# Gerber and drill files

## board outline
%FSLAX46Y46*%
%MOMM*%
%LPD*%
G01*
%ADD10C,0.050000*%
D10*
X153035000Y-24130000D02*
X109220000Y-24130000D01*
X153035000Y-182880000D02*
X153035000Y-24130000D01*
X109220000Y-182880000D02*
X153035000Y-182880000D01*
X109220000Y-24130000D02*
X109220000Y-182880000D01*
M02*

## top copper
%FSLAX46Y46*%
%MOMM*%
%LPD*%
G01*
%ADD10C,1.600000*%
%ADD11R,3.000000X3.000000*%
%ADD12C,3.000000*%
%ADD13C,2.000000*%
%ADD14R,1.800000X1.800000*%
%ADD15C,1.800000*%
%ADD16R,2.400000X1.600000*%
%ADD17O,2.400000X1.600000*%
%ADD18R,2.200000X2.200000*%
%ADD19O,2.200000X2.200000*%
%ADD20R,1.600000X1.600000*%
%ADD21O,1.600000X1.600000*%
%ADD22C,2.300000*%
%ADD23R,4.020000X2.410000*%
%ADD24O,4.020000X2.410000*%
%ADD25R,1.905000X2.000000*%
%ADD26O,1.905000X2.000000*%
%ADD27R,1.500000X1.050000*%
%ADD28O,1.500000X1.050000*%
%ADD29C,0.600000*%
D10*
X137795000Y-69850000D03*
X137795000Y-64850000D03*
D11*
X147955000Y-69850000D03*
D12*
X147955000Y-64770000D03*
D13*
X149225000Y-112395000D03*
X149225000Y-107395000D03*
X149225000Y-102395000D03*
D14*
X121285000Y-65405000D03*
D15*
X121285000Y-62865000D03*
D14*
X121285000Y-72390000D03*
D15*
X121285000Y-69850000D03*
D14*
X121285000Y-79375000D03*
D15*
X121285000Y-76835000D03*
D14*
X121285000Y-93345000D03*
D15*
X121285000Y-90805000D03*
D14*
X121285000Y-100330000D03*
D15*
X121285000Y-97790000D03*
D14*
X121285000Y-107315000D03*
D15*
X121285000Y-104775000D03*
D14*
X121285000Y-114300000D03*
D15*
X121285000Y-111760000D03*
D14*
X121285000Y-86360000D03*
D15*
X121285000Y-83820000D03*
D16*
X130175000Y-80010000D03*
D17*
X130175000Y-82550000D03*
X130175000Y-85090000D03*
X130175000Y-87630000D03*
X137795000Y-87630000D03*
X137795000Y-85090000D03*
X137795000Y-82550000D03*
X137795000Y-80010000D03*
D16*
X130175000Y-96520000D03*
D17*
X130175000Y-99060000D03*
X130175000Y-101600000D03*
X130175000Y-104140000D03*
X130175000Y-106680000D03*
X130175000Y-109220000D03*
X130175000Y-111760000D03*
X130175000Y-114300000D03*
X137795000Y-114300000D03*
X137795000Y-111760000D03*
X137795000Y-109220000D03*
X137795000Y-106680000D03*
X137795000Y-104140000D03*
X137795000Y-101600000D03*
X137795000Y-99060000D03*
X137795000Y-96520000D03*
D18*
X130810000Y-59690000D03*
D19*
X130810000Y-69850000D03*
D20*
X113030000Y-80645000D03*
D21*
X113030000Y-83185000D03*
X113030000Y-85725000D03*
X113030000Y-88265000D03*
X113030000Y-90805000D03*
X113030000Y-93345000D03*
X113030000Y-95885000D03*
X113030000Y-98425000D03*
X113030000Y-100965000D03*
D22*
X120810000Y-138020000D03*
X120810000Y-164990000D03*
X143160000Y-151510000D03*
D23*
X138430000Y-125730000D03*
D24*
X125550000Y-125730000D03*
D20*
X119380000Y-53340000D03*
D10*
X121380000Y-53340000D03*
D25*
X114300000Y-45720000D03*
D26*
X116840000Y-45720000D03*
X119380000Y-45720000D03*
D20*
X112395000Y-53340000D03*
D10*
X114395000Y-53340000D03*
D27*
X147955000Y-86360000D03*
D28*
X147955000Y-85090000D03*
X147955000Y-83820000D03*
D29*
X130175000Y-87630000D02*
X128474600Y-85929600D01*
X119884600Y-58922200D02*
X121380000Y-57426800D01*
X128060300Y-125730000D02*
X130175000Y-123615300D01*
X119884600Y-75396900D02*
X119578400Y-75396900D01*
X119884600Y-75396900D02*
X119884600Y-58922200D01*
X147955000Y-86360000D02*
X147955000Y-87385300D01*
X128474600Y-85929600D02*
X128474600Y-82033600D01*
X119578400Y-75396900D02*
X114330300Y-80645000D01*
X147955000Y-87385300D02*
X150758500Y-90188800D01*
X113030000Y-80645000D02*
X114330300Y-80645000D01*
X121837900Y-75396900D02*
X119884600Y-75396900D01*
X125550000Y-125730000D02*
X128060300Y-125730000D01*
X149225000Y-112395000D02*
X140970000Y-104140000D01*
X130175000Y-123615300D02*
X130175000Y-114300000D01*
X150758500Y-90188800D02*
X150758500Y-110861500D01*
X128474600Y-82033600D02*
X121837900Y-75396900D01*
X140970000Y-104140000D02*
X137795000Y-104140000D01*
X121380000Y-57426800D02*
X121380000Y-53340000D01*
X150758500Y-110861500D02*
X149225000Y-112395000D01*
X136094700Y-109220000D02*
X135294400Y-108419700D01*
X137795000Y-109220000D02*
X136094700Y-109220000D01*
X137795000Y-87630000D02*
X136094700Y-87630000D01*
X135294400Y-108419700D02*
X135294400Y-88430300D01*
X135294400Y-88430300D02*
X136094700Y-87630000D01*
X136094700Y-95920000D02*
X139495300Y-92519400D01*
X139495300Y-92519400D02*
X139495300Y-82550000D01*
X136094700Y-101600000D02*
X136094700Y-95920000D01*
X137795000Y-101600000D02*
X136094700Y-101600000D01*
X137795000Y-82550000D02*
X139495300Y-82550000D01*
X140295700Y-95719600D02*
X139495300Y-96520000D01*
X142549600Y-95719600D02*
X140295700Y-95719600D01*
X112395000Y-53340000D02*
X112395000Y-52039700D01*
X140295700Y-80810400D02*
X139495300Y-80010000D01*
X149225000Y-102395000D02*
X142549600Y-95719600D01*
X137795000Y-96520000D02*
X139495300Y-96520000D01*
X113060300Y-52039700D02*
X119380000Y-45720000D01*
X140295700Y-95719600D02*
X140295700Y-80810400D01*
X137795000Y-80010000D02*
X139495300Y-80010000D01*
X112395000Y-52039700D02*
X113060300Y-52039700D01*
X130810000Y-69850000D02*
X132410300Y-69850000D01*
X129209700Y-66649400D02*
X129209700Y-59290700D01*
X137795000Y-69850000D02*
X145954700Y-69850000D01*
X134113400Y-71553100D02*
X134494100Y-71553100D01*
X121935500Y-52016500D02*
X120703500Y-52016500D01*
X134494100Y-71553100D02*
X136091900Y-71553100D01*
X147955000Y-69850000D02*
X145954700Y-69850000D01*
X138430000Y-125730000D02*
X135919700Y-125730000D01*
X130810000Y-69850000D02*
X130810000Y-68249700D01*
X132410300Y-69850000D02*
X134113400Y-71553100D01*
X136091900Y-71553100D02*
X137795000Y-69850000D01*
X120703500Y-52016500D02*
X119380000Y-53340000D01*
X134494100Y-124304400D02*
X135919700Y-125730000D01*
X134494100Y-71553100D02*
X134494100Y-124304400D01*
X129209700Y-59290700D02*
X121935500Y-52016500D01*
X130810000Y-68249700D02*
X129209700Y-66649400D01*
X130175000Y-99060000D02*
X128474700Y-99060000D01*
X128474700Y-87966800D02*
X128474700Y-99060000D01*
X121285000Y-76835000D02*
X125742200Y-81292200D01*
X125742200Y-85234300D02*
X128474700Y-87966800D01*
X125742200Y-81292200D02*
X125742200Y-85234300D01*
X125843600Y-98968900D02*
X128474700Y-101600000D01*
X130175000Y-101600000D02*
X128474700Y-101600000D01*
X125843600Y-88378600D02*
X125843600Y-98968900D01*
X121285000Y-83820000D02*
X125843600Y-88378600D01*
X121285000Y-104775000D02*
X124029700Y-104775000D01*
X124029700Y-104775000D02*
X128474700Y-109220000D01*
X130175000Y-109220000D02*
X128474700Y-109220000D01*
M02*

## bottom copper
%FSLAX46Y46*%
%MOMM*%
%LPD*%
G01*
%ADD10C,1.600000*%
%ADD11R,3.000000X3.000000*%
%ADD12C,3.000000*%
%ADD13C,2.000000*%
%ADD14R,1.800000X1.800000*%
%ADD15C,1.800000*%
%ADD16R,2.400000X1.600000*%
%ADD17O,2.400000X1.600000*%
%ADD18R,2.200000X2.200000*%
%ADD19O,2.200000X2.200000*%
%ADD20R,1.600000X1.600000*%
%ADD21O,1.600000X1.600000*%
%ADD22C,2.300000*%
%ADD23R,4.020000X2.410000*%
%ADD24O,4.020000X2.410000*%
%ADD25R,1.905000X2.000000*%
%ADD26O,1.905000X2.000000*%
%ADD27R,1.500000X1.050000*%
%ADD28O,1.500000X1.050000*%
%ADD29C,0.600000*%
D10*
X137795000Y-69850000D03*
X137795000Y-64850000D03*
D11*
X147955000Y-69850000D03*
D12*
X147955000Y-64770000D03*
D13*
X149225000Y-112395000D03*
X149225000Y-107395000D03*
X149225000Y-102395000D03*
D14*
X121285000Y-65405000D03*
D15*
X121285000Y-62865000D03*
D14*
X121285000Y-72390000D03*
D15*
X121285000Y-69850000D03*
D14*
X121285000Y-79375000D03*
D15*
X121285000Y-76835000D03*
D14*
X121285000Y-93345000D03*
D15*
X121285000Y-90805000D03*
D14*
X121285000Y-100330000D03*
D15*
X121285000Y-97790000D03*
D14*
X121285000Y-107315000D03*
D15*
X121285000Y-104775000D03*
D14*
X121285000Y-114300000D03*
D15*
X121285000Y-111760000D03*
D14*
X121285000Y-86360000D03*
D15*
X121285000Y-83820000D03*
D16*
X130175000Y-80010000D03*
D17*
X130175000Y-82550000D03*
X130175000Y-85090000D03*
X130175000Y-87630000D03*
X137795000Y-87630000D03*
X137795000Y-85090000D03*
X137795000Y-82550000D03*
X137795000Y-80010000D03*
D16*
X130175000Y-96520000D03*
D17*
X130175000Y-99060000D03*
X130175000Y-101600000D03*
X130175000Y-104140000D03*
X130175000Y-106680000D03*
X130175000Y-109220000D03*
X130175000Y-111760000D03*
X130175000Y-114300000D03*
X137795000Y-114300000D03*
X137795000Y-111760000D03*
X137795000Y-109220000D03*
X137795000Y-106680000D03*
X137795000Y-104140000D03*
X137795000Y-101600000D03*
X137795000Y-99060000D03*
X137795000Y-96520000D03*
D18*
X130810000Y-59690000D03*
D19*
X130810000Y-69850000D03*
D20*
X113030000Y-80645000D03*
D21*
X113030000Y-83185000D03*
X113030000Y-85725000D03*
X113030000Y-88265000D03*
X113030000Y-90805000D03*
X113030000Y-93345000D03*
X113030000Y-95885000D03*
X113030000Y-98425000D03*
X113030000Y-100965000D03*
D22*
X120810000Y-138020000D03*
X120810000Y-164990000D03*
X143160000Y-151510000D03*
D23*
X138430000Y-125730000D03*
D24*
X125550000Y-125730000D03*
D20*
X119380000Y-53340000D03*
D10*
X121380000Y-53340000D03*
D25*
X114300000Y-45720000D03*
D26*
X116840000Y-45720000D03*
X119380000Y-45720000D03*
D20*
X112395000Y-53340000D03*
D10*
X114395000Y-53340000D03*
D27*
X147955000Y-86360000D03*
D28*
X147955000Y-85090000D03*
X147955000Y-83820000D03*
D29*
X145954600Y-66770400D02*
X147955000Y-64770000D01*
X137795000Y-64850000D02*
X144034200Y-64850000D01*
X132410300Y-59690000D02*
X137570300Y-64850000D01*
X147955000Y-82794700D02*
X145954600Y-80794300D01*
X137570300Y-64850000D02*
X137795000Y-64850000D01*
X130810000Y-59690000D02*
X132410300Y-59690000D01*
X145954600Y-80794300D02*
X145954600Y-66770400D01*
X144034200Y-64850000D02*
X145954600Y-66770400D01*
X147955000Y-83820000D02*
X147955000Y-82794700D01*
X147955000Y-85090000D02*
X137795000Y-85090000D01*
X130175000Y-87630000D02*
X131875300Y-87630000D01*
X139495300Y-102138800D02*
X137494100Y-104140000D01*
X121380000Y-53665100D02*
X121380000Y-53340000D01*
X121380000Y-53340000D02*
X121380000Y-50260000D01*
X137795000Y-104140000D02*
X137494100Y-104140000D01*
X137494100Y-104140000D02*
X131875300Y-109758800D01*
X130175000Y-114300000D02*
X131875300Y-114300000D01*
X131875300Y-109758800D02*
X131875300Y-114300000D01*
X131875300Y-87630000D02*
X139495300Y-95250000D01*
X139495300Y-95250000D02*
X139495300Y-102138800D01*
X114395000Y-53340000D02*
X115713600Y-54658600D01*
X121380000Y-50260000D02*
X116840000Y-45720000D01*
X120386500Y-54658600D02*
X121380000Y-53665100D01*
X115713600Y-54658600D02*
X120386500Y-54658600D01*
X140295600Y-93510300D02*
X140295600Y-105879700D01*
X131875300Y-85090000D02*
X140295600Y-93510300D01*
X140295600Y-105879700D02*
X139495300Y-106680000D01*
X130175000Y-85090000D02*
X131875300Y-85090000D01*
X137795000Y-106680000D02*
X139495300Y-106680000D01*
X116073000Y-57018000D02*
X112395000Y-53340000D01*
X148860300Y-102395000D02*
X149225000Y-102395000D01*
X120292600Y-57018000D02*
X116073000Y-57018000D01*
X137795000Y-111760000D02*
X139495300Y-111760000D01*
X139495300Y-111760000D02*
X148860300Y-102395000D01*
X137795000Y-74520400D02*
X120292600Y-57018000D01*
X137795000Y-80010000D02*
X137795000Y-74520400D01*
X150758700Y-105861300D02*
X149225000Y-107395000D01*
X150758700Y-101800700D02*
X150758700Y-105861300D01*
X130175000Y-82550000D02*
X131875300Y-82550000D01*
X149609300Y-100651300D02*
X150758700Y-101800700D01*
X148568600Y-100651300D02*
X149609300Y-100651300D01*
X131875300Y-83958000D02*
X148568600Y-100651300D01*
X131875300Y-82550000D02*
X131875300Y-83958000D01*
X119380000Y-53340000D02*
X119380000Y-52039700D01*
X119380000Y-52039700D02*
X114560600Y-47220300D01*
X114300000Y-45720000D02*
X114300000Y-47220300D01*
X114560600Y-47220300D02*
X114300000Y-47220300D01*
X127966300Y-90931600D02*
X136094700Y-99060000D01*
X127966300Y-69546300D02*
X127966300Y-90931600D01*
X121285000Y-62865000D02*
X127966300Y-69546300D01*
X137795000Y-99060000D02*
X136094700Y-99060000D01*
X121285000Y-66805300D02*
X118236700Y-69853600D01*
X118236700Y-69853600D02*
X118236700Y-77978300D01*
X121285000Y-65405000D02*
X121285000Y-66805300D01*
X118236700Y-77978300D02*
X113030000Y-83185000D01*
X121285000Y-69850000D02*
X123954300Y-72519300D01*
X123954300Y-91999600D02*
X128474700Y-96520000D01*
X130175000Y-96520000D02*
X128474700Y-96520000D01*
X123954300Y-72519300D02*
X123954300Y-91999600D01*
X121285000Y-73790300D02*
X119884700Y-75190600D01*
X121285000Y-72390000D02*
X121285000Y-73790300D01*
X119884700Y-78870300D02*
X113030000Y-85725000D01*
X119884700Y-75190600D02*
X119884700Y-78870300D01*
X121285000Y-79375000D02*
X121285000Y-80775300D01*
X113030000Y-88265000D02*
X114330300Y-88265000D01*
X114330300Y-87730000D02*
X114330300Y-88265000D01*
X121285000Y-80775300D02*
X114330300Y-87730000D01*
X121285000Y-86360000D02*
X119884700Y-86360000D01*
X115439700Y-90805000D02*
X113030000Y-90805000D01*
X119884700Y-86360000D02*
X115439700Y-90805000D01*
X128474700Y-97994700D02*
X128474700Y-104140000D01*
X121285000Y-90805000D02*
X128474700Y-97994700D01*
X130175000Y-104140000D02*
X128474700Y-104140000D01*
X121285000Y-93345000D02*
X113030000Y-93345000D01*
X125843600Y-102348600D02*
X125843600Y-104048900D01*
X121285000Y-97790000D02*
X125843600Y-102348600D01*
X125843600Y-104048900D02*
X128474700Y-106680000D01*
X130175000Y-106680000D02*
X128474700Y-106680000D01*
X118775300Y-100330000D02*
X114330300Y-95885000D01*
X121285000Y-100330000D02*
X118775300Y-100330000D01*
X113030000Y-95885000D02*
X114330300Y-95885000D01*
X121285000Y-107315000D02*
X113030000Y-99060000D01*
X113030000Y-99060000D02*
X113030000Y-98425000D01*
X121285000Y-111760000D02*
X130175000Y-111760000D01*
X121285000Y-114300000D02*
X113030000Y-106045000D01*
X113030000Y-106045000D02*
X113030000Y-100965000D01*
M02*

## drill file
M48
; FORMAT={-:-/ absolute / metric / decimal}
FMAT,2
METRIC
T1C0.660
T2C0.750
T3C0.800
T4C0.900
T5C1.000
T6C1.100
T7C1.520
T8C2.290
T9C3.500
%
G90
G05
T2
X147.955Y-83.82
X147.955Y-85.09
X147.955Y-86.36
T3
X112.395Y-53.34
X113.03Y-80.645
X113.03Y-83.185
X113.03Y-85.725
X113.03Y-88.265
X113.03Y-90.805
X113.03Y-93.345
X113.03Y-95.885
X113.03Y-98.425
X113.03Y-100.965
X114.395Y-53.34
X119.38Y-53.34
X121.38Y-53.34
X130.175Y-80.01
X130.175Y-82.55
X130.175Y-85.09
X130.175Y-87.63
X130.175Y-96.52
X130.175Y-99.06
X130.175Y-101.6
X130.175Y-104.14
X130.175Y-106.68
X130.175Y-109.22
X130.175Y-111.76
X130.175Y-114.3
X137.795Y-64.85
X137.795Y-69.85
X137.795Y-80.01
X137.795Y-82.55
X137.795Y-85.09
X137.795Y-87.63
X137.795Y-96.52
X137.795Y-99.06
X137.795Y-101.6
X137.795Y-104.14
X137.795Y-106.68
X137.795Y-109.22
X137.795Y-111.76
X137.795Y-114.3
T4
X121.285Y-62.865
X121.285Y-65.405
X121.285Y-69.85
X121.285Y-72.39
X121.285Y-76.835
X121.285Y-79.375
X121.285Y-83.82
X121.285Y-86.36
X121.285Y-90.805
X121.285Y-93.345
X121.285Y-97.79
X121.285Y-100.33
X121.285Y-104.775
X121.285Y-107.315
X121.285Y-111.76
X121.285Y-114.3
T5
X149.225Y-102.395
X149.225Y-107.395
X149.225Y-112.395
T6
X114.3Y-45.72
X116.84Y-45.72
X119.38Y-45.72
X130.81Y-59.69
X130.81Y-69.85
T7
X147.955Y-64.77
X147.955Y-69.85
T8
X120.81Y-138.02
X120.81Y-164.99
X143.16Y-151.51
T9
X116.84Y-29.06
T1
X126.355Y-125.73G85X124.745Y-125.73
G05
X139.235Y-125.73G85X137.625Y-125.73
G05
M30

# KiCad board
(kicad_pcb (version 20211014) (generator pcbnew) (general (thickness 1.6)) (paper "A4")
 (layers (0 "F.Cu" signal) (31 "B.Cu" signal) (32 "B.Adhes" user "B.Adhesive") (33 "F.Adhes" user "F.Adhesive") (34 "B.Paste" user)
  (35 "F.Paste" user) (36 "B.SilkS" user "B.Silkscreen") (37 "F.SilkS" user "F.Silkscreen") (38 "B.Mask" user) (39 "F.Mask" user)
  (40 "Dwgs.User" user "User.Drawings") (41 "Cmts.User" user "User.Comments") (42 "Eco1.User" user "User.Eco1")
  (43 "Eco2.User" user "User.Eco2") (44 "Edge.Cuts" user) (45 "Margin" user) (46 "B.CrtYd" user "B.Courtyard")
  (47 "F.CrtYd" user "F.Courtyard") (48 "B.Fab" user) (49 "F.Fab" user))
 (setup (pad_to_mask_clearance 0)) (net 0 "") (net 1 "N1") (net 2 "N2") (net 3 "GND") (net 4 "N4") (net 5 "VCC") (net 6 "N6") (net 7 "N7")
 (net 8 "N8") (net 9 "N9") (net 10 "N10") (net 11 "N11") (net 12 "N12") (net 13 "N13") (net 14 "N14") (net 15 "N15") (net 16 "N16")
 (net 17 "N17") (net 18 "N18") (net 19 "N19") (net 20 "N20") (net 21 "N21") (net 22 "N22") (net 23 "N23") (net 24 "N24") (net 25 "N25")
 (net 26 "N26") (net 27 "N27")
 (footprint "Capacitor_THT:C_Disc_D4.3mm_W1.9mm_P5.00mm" (layer "F.Cu") (at 137.795 69.85 90)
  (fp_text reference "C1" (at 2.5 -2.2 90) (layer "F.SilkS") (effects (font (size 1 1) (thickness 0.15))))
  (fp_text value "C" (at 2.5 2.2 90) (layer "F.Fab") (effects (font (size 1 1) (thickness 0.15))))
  (pad "1" thru_hole circle locked (at 0 0 90) (size 1.6 1.6) (drill 0.8) (layers *.Cu *.Mask) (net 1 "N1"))
  (pad "2" thru_hole circle locked (at 5 0 90) (size 1.6 1.6) (drill 0.8) (layers *.Cu *.Mask) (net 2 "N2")))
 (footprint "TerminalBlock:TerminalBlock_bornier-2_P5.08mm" (layer "F.Cu") (at 147.955 69.85 90)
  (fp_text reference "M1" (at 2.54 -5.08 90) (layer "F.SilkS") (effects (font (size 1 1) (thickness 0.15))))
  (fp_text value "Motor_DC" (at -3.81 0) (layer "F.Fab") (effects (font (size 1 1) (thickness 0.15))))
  (pad "1" thru_hole rect locked (at 0 0 90) (size 3 3) (drill 1.52) (layers *.Cu *.Mask) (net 1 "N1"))
  (pad "2" thru_hole circle locked (at 5.08 0 90) (size 3 3) (drill 1.52) (layers *.Cu *.Mask) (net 2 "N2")))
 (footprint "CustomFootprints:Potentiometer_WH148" (layer "F.Cu") (at 140.335 107.395 90)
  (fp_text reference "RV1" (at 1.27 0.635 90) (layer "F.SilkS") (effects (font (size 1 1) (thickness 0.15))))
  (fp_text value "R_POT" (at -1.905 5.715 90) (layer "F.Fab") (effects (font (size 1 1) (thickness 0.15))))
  (pad "1" thru_hole circle locked (at -5 8.89 90) (size 2 2) (drill 1) (layers *.Cu *.Mask) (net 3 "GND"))
  (pad "2" thru_hole circle locked (at 0 8.89 90) (size 2 2) (drill 1) (layers *.Cu *.Mask) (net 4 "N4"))
  (pad "3" thru_hole circle locked (at 5 8.89 90) (size 2 2) (drill 1) (layers *.Cu *.Mask) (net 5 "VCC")))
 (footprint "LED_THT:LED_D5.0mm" (layer "F.Cu") (at 121.285 65.405 90)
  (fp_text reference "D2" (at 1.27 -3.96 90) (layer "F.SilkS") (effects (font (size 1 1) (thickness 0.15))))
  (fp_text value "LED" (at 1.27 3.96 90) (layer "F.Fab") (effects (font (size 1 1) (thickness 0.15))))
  (pad "1" thru_hole rect locked (at 0 0 90) (size 1.8 1.8) (drill 0.9) (layers *.Cu *.Mask) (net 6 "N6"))
  (pad "2" thru_hole circle locked (at 2.54 0 90) (size 1.8 1.8) (drill 0.9) (layers *.Cu *.Mask) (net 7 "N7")))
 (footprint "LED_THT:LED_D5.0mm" (layer "F.Cu") (at 121.285 72.39 90)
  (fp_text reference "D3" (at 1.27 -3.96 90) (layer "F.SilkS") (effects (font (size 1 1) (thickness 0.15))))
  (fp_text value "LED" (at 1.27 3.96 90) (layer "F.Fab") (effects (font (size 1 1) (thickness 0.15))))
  (pad "1" thru_hole rect locked (at 0 0 90) (size 1.8 1.8) (drill 0.9) (layers *.Cu *.Mask) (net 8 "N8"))
  (pad "2" thru_hole circle locked (at 2.54 0 90) (size 1.8 1.8) (drill 0.9) (layers *.Cu *.Mask) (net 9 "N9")))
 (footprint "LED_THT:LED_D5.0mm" (layer "F.Cu") (at 121.285 79.375 90)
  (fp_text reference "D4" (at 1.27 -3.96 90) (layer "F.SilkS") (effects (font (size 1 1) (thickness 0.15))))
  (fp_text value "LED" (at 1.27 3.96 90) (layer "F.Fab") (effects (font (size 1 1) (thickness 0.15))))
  (pad "1" thru_hole rect locked (at 0 0 90) (size 1.8 1.8) (drill 0.9) (layers *.Cu *.Mask) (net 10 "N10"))
  (pad "2" thru_hole circle locked (at 2.54 0 90) (size 1.8 1.8) (drill 0.9) (layers *.Cu *.Mask) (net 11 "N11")))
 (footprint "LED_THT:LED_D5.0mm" (layer "F.Cu") (at 121.285 93.345 90)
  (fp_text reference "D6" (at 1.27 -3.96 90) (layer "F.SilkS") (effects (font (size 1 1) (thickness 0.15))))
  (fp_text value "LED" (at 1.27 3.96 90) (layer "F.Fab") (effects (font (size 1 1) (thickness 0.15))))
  (pad "1" thru_hole rect locked (at 0 0 90) (size 1.8 1.8) (drill 0.9) (layers *.Cu *.Mask) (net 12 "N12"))
  (pad "2" thru_hole circle locked (at 2.54 0 90) (size 1.8 1.8) (drill 0.9) (layers *.Cu *.Mask) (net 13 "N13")))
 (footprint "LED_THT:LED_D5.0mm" (layer "F.Cu") (at 121.285 100.33 90)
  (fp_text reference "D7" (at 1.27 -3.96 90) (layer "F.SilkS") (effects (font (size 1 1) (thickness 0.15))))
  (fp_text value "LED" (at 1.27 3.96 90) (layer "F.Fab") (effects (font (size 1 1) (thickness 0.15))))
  (pad "1" thru_hole rect locked (at 0 0 90) (size 1.8 1.8) (drill 0.9) (layers *.Cu *.Mask) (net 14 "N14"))
  (pad "2" thru_hole circle locked (at 2.54 0 90) (size 1.8 1.8) (drill 0.9) (layers *.Cu *.Mask) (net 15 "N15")))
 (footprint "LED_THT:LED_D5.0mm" (layer "F.Cu") (at 121.285 107.315 90)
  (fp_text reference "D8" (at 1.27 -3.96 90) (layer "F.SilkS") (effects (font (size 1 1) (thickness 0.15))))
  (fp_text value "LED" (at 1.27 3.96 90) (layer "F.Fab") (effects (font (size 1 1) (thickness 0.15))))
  (pad "1" thru_hole rect locked (at 0 0 90) (size 1.8 1.8) (drill 0.9) (layers *.Cu *.Mask) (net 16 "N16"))
  (pad "2" thru_hole circle locked (at 2.54 0 90) (size 1.8 1.8) (drill 0.9) (layers *.Cu *.Mask) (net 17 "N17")))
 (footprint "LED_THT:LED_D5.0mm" (layer "F.Cu") (at 121.285 114.3 90)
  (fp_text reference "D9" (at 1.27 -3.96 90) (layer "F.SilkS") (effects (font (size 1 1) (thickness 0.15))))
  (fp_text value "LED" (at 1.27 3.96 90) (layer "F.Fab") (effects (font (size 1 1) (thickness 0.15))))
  (pad "1" thru_hole rect locked (at 0 0 90) (size 1.8 1.8) (drill 0.9) (layers *.Cu *.Mask) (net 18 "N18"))
  (pad "2" thru_hole circle locked (at 2.54 0 90) (size 1.8 1.8) (drill 0.9) (layers *.Cu *.Mask) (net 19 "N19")))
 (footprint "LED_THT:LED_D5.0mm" (layer "F.Cu") (at 121.285 86.36 90)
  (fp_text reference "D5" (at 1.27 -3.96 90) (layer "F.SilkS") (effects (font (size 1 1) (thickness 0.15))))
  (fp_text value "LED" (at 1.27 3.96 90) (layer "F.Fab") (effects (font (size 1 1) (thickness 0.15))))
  (pad "1" thru_hole rect locked (at 0 0 90) (size 1.8 1.8) (drill 0.9) (layers *.Cu *.Mask) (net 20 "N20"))
  (pad "2" thru_hole circle locked (at 2.54 0 90) (size 1.8 1.8) (drill 0.9) (layers *.Cu *.Mask) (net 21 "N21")))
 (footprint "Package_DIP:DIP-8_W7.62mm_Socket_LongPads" (layer "F.Cu") (at 130.175 80.01)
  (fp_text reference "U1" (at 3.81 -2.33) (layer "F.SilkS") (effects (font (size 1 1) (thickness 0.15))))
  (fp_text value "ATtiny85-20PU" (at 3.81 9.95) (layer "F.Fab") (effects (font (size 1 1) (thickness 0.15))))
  (pad "1" thru_hole rect locked (at 0 0) (size 2.4 1.6) (drill 0.8) (layers *.Cu *.Mask) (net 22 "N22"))
  (pad "2" thru_hole oval locked (at 0 2.54) (size 2.4 1.6) (drill 0.8) (layers *.Cu *.Mask) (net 4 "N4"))
  (pad "3" thru_hole oval locked (at 0 5.08) (size 2.4 1.6) (drill 0.8) (layers *.Cu *.Mask) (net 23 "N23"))
  (pad "4" thru_hole oval locked (at 0 7.62) (size 2.4 1.6) (drill 0.8) (layers *.Cu *.Mask) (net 3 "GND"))
  (pad "5" thru_hole oval locked (at 7.62 7.62) (size 2.4 1.6) (drill 0.8) (layers *.Cu *.Mask) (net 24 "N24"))
  (pad "6" thru_hole oval locked (at 7.62 5.08) (size 2.4 1.6) (drill 0.8) (layers *.Cu *.Mask) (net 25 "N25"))
  (pad "7" thru_hole oval locked (at 7.62 2.54) (size 2.4 1.6) (drill 0.8) (layers *.Cu *.Mask) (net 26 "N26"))
  (pad "8" thru_hole oval locked (at 7.62 0) (size 2.4 1.6) (drill 0.8) (layers *.Cu *.Mask) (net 5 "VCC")))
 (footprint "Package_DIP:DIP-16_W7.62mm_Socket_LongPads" (layer "F.Cu") (at 130.175 96.52)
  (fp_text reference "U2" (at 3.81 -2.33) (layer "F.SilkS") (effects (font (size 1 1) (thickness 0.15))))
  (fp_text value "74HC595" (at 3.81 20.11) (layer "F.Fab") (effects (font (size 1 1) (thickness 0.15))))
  (pad "1" thru_hole rect locked (at 0 0) (size 2.4 1.6) (drill 0.8) (layers *.Cu *.Mask) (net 9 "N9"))
  (pad "2" thru_hole oval locked (at 0 2.54) (size 2.4 1.6) (drill 0.8) (layers *.Cu *.Mask) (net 11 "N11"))
  (pad "3" thru_hole oval locked (at 0 5.08) (size 2.4 1.6) (drill 0.8) (layers *.Cu *.Mask) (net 21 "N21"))
  (pad "4" thru_hole oval locked (at 0 7.62) (size 2.4 1.6) (drill 0.8) (layers *.Cu *.Mask) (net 13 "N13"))
  (pad "5" thru_hole oval locked (at 0 10.16) (size 2.4 1.6) (drill 0.8) (layers *.Cu *.Mask) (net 15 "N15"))
  (pad "6" thru_hole oval locked (at 0 12.7) (size 2.4 1.6) (drill 0.8) (layers *.Cu *.Mask) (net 17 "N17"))
  (pad "7" thru_hole oval locked (at 0 15.24) (size 2.4 1.6) (drill 0.8) (layers *.Cu *.Mask) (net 19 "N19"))
  (pad "8" thru_hole oval locked (at 0 17.78) (size 2.4 1.6) (drill 0.8) (layers *.Cu *.Mask) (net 3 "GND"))
  (pad "9" thru_hole oval locked (at 7.62 17.78) (size 2.4 1.6) (drill 0.8) (layers *.Cu *.Mask) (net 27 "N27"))
  (pad "10" thru_hole oval locked (at 7.62 15.24) (size 2.4 1.6) (drill 0.8) (layers *.Cu *.Mask) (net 5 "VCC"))
  (pad "11" thru_hole oval locked (at 7.62 12.7) (size 2.4 1.6) (drill 0.8) (layers *.Cu *.Mask) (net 24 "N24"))
  (pad "12" thru_hole oval locked (at 7.62 10.16) (size 2.4 1.6) (drill 0.8) (layers *.Cu *.Mask) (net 23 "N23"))
  (pad "13" thru_hole oval locked (at 7.62 7.62) (size 2.4 1.6) (drill 0.8) (layers *.Cu *.Mask) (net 3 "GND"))
  (pad "14" thru_hole oval locked (at 7.62 5.08) (size 2.4 1.6) (drill 0.8) (layers *.Cu *.Mask) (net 26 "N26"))
  (pad "15" thru_hole oval locked (at 7.62 2.54) (size 2.4 1.6) (drill 0.8) (layers *.Cu *.Mask) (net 7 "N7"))
  (pad "16" thru_hole oval locked (at 7.62 0) (size 2.4 1.6) (drill 0.8) (layers *.Cu *.Mask) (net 5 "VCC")))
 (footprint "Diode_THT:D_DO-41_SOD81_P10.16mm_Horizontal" (layer "F.Cu") (at 130.81 59.69 -90)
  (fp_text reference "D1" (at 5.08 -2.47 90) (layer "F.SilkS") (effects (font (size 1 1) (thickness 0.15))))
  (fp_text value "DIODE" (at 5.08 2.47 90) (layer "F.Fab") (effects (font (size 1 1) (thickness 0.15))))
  (pad "1" thru_hole rect locked (at 0 0 270) (size 2.2 2.2) (drill 1.1) (layers *.Cu *.Mask) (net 2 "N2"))
  (pad "2" thru_hole oval locked (at 10.16 0 270) (size 2.2 2.2) (drill 1.1) (layers *.Cu *.Mask) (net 1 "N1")))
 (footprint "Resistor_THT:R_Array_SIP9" (layer "F.Cu") (at 113.03 80.645 -90)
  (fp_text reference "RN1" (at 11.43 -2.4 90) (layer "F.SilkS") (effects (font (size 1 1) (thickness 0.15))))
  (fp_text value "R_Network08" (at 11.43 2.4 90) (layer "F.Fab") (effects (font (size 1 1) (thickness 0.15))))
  (pad "1" thru_hole rect locked (at 0 0 270) (size 1.6 1.6) (drill 0.8) (layers *.Cu *.Mask) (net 3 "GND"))
  (pad "2" thru_hole oval locked (at 2.54 0 270) (size 1.6 1.6) (drill 0.8) (layers *.Cu *.Mask) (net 6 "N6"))
  (pad "3" thru_hole oval locked (at 5.08 0 270) (size 1.6 1.6) (drill 0.8) (layers *.Cu *.Mask) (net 8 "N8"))
  (pad "4" thru_hole oval locked (at 7.62 0 270) (size 1.6 1.6) (drill 0.8) (layers *.Cu *.Mask) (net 10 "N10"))
  (pad "5" thru_hole oval locked (at 10.16 0 270) (size 1.6 1.6) (drill 0.8) (layers *.Cu *.Mask) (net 20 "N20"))
  (pad "6" thru_hole oval locked (at 12.7 0 270) (size 1.6 1.6) (drill 0.8) (layers *.Cu *.Mask) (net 12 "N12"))
  (pad "7" thru_hole oval locked (at 15.24 0 270) (size 1.6 1.6) (drill 0.8) (layers *.Cu *.Mask) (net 14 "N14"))
  (pad "8" thru_hole oval locked (at 17.78 0 270) (size 1.6 1.6) (drill 0.8) (layers *.Cu *.Mask) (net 16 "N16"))
  (pad "9" thru_hole oval locked (at 20.32 0 270) (size 1.6 1.6) (drill 0.8) (layers *.Cu *.Mask) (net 18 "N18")))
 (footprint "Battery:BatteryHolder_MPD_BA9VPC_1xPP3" (layer "F.Cu") (at 138.43 125.73 -90)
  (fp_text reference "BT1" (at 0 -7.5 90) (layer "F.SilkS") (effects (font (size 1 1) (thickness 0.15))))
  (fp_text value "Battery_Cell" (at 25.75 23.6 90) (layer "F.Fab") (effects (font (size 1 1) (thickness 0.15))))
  (pad "" np_thru_hole circle locked (at 12.29 17.62 270) (size 2.3 2.3) (drill 2.29) (layers *.Cu *.Mask))
  (pad "" np_thru_hole circle locked (at 39.26 17.62 270) (size 2.3 2.3) (drill 2.29) (layers *.Cu *.Mask))
  (pad "" np_thru_hole circle locked (at 25.78 -4.73 270) (size 2.3 2.3) (drill 2.29) (layers *.Cu *.Mask))
  (pad "1" thru_hole rect locked (at 0 0 270) (size 2.41 4.02) (drill oval 0.66 2.27) (layers *.Cu *.Mask) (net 1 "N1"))
  (pad "2" thru_hole oval locked (at 0 12.88 270) (size 2.41 4.02) (drill oval 0.66 2.27) (layers *.Cu *.Mask) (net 3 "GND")))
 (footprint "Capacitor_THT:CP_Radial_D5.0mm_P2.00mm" (layer "F.Cu") (at 119.38 53.34)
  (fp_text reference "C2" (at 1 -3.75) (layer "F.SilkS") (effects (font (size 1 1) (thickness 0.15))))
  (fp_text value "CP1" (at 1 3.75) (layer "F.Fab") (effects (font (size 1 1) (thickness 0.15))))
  (pad "1" thru_hole rect locked (at 0 0) (size 1.6 1.6) (drill 0.8) (layers *.Cu *.Mask) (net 1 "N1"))
  (pad "2" thru_hole circle locked (at 2 0) (size 1.6 1.6) (drill 0.8) (layers *.Cu *.Mask) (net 3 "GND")))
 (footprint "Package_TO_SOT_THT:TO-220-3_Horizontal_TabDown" (layer "F.Cu") (at 114.3 45.72)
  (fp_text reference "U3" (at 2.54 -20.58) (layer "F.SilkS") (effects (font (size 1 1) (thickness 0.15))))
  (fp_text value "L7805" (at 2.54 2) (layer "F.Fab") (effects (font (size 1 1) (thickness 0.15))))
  (pad "" np_thru_hole oval locked (at 2.54 -16.66) (size 3.5 3.5) (drill 3.5) (layers *.Cu *.Mask))
  (pad "1" thru_hole rect locked (at 0 0) (size 1.905 2) (drill 1.1) (layers *.Cu *.Mask) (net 1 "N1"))
  (pad "2" thru_hole oval locked (at 2.54 0) (size 1.905 2) (drill 1.1) (layers *.Cu *.Mask) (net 3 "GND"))
  (pad "3" thru_hole oval locked (at 5.08 0) (size 1.905 2) (drill 1.1) (layers *.Cu *.Mask) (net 5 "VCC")))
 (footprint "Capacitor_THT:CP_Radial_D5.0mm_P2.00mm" (layer "F.Cu") (at 112.395 53.34)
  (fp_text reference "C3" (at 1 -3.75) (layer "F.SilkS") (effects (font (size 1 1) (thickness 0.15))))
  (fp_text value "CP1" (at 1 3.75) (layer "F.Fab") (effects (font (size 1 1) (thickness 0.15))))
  (pad "1" thru_hole rect locked (at 0 0) (size 1.6 1.6) (drill 0.8) (layers *.Cu *.Mask) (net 5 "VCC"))
  (pad "2" thru_hole circle locked (at 2 0) (size 1.6 1.6) (drill 0.8) (layers *.Cu *.Mask) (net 3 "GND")))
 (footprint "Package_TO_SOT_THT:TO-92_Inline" (layer "F.Cu") (at 147.955 86.36 90)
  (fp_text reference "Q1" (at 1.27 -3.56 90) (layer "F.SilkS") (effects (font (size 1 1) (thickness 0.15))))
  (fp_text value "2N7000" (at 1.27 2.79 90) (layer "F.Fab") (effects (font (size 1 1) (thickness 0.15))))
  (pad "1" thru_hole rect locked (at 0 0 90) (size 1.05 1.5) (drill 0.75) (layers *.Cu *.Mask) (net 3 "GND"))
  (pad "2" thru_hole oval locked (at 1.27 0 90) (size 1.05 1.5) (drill 0.75) (layers *.Cu *.Mask) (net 25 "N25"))
  (pad "3" thru_hole oval locked (at 2.54 0 90) (size 1.05 1.5) (drill 0.75) (layers *.Cu *.Mask) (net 2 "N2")))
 (gr_line (start 153.035 24.13) (end 109.22 24.13) (layer "Edge.Cuts") (width 0.05))
 (gr_line (start 153.035 182.88) (end 153.035 24.13) (layer "Edge.Cuts") (width 0.05))
 (gr_line (start 109.22 182.88) (end 153.035 182.88) (layer "Edge.Cuts") (width 0.05))
 (gr_line (start 109.22 24.13) (end 109.22 182.88) (layer "Edge.Cuts") (width 0.05))
 (segment (start 145.9546 66.7704) (end 147.955 64.77) (width 0.6) (layer "B.Cu") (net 2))
 (segment (start 137.795 64.85) (end 144.0342 64.85) (width 0.6) (layer "B.Cu") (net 2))
 (segment (start 132.4103 59.69) (end 137.5703 64.85) (width 0.6) (layer "B.Cu") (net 2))
 (segment (start 147.955 82.7947) (end 145.9546 80.7943) (width 0.6) (layer "B.Cu") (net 2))
 (segment (start 137.5703 64.85) (end 137.795 64.85) (width 0.6) (layer "B.Cu") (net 2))
 (segment (start 130.81 59.69) (end 132.4103 59.69) (width 0.6) (layer "B.Cu") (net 2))
 (segment (start 145.9546 80.7943) (end 145.9546 66.7704) (width 0.6) (layer "B.Cu") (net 2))
 (segment (start 144.0342 64.85) (end 145.9546 66.7704) (width 0.6) (layer "B.Cu") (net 2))
 (segment (start 147.955 83.82) (end 147.955 82.7947) (width 0.6) (layer "B.Cu") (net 2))
 (segment (start 147.955 85.09) (end 137.795 85.09) (width 0.6) (layer "B.Cu") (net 25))
 (segment (start 130.175 87.63) (end 128.4746 85.9296) (width 0.6) (layer "F.Cu") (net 3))
 (segment (start 119.8846 58.9222) (end 121.38 57.4268) (width 0.6) (layer "F.Cu") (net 3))
 (segment (start 128.0603 125.73) (end 130.175 123.6153) (width 0.6) (layer "F.Cu") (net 3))
 (segment (start 119.8846 75.3969) (end 119.5784 75.3969) (width 0.6) (layer "F.Cu") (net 3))
 (segment (start 119.8846 75.3969) (end 119.8846 58.9222) (width 0.6) (layer "F.Cu") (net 3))
 (segment (start 147.955 86.36) (end 147.955 87.3853) (width 0.6) (layer "F.Cu") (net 3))
 (segment (start 128.4746 85.9296) (end 128.4746 82.0336) (width 0.6) (layer "F.Cu") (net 3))
 (segment (start 119.5784 75.3969) (end 114.3303 80.645) (width 0.6) (layer "F.Cu") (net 3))
 (segment (start 147.955 87.3853) (end 150.7585 90.1888) (width 0.6) (layer "F.Cu") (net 3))
 (segment (start 113.03 80.645) (end 114.3303 80.645) (width 0.6) (layer "F.Cu") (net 3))
 (segment (start 121.8379 75.3969) (end 119.8846 75.3969) (width 0.6) (layer "F.Cu") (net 3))
 (segment (start 125.55 125.73) (end 128.0603 125.73) (width 0.6) (layer "F.Cu") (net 3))
 (segment (start 149.225 112.395) (end 140.97 104.14) (width 0.6) (layer "F.Cu") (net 3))
 (segment (start 130.175 123.6153) (end 130.175 114.3) (width 0.6) (layer "F.Cu") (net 3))
 (segment (start 150.7585 90.1888) (end 150.7585 110.8615) (width 0.6) (layer "F.Cu") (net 3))
 (segment (start 128.4746 82.0336) (end 121.8379 75.3969) (width 0.6) (layer "F.Cu") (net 3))
 (segment (start 140.97 104.14) (end 137.795 104.14) (width 0.6) (layer "F.Cu") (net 3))
 (segment (start 121.38 57.4268) (end 121.38 53.34) (width 0.6) (layer "F.Cu") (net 3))
 (segment (start 150.7585 110.8615) (end 149.225 112.395) (width 0.6) (layer "F.Cu") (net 3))
 (segment (start 130.175 87.63) (end 131.8753 87.63) (width 0.6) (layer "B.Cu") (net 3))
 (segment (start 139.4953 102.1388) (end 137.4941 104.14) (width 0.6) (layer "B.Cu") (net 3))
 (segment (start 121.38 53.6651) (end 121.38 53.34) (width 0.6) (layer "B.Cu") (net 3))
 (segment (start 121.38 53.34) (end 121.38 50.26) (width 0.6) (layer "B.Cu") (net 3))
 (segment (start 137.795 104.14) (end 137.4941 104.14) (width 0.6) (layer "B.Cu") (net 3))
 (segment (start 137.4941 104.14) (end 131.8753 109.7588) (width 0.6) (layer "B.Cu") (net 3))
 (segment (start 130.175 114.3) (end 131.8753 114.3) (width 0.6) (layer "B.Cu") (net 3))
 (segment (start 131.8753 109.7588) (end 131.8753 114.3) (width 0.6) (layer "B.Cu") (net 3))
 (segment (start 131.8753 87.63) (end 139.4953 95.25) (width 0.6) (layer "B.Cu") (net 3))
 (segment (start 139.4953 95.25) (end 139.4953 102.1388) (width 0.6) (layer "B.Cu") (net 3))
 (segment (start 114.395 53.34) (end 115.7136 54.6586) (width 0.6) (layer "B.Cu") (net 3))
 (segment (start 121.38 50.26) (end 116.84 45.72) (width 0.6) (layer "B.Cu") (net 3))
 (segment (start 120.3865 54.6586) (end 121.38 53.6651) (width 0.6) (layer "B.Cu") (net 3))
 (segment (start 115.7136 54.6586) (end 120.3865 54.6586) (width 0.6) (layer "B.Cu") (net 3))
 (segment (start 136.0947 109.22) (end 135.2944 108.4197) (width 0.6) (layer "F.Cu") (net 24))
 (segment (start 137.795 109.22) (end 136.0947 109.22) (width 0.6) (layer "F.Cu") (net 24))
 (segment (start 137.795 87.63) (end 136.0947 87.63) (width 0.6) (layer "F.Cu") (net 24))
 (segment (start 135.2944 108.4197) (end 135.2944 88.4303) (width 0.6) (layer "F.Cu") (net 24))
 (segment (start 135.2944 88.4303) (end 136.0947 87.63) (width 0.6) (layer "F.Cu") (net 24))
 (segment (start 140.2956 93.5103) (end 140.2956 105.8797) (width 0.6) (layer "B.Cu") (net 23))
 (segment (start 131.8753 85.09) (end 140.2956 93.5103) (width 0.6) (layer "B.Cu") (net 23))
 (segment (start 140.2956 105.8797) (end 139.4953 106.68) (width 0.6) (layer "B.Cu") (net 23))
 (segment (start 130.175 85.09) (end 131.8753 85.09) (width 0.6) (layer "B.Cu") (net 23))
 (segment (start 137.795 106.68) (end 139.4953 106.68) (width 0.6) (layer "B.Cu") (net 23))
 (segment (start 136.0947 95.92) (end 139.4953 92.5194) (width 0.6) (layer "F.Cu") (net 26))
 (segment (start 139.4953 92.5194) (end 139.4953 82.55) (width 0.6) (layer "F.Cu") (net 26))
 (segment (start 136.0947 101.6) (end 136.0947 95.92) (width 0.6) (layer "F.Cu") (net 26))
 (segment (start 137.795 101.6) (end 136.0947 101.6) (width 0.6) (layer "F.Cu") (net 26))
 (segment (start 137.795 82.55) (end 139.4953 82.55) (width 0.6) (layer "F.Cu") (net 26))
 (segment (start 140.2957 95.7196) (end 139.4953 96.52) (width 0.6) (layer "F.Cu") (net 5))
 (segment (start 142.5496 95.7196) (end 140.2957 95.7196) (width 0.6) (layer "F.Cu") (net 5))
 (segment (start 112.395 53.34) (end 112.395 52.0397) (width 0.6) (layer "F.Cu") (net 5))
 (segment (start 140.2957 80.8104) (end 139.4953 80.01) (width 0.6) (layer "F.Cu") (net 5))
 (segment (start 149.225 102.395) (end 142.5496 95.7196) (width 0.6) (layer "F.Cu") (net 5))
 (segment (start 137.795 96.52) (end 139.4953 96.52) (width 0.6) (layer "F.Cu") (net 5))
 (segment (start 113.0603 52.0397) (end 119.38 45.72) (width 0.6) (layer "F.Cu") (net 5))
 (segment (start 140.2957 95.7196) (end 140.2957 80.8104) (width 0.6) (layer "F.Cu") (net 5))
 (segment (start 137.795 80.01) (end 139.4953 80.01) (width 0.6) (layer "F.Cu") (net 5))
 (segment (start 112.395 52.0397) (end 113.0603 52.0397) (width 0.6) (layer "F.Cu") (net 5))
 (segment (start 116.073 57.018) (end 112.395 53.34) (width 0.6) (layer "B.Cu") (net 5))
 (segment (start 148.8603 102.395) (end 149.225 102.395) (width 0.6) (layer "B.Cu") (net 5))
 (segment (start 120.2926 57.018) (end 116.073 57.018) (width 0.6) (layer "B.Cu") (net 5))
 (segment (start 137.795 111.76) (end 139.4953 111.76) (width 0.6) (layer "B.Cu") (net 5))
 (segment (start 139.4953 111.76) (end 148.8603 102.395) (width 0.6) (layer "B.Cu") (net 5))
 (segment (start 137.795 74.5204) (end 120.2926 57.018) (width 0.6) (layer "B.Cu") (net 5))
 (segment (start 137.795 80.01) (end 137.795 74.5204) (width 0.6) (layer "B.Cu") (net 5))
 (segment (start 150.7587 105.8613) (end 149.225 107.395) (width 0.6) (layer "B.Cu") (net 4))
 (segment (start 150.7587 101.8007) (end 150.7587 105.8613) (width 0.6) (layer "B.Cu") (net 4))
 (segment (start 130.175 82.55) (end 131.8753 82.55) (width 0.6) (layer "B.Cu") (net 4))
 (segment (start 149.6093 100.6513) (end 150.7587 101.8007) (width 0.6) (layer "B.Cu") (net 4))
 (segment (start 148.5686 100.6513) (end 149.6093 100.6513) (width 0.6) (layer "B.Cu") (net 4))
 (segment (start 131.8753 83.958) (end 148.5686 100.6513) (width 0.6) (layer "B.Cu") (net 4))
 (segment (start 131.8753 82.55) (end 131.8753 83.958) (width 0.6) (layer "B.Cu") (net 4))
 (segment (start 130.81 69.85) (end 132.4103 69.85) (width 0.6) (layer "F.Cu") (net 1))
 (segment (start 129.2097 66.6494) (end 129.2097 59.2907) (width 0.6) (layer "F.Cu") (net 1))
 (segment (start 137.795 69.85) (end 145.9547 69.85) (width 0.6) (layer "F.Cu") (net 1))
 (segment (start 134.1134 71.5531) (end 134.4941 71.5531) (width 0.6) (layer "F.Cu") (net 1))
 (segment (start 121.9355 52.0165) (end 120.7035 52.0165) (width 0.6) (layer "F.Cu") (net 1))
 (segment (start 134.4941 71.5531) (end 136.0919 71.5531) (width 0.6) (layer "F.Cu") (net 1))
 (segment (start 147.955 69.85) (end 145.9547 69.85) (width 0.6) (layer "F.Cu") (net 1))
 (segment (start 138.43 125.73) (end 135.9197 125.73) (width 0.6) (layer "F.Cu") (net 1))
 (segment (start 130.81 69.85) (end 130.81 68.2497) (width 0.6) (layer "F.Cu") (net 1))
 (segment (start 132.4103 69.85) (end 134.1134 71.5531) (width 0.6) (layer "F.Cu") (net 1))
 (segment (start 136.0919 71.5531) (end 137.795 69.85) (width 0.6) (layer "F.Cu") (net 1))
 (segment (start 120.7035 52.0165) (end 119.38 53.34) (width 0.6) (layer "F.Cu") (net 1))
 (segment (start 134.4941 124.3044) (end 135.9197 125.73) (width 0.6) (layer "F.Cu") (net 1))
 (segment (start 134.4941 71.5531) (end 134.4941 124.3044) (width 0.6) (layer "F.Cu") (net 1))
 (segment (start 129.2097 59.2907) (end 121.9355 52.0165) (width 0.6) (layer "F.Cu") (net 1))
 (segment (start 130.81 68.2497) (end 129.2097 66.6494) (width 0.6) (layer "F.Cu") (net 1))
 (segment (start 119.38 53.34) (end 119.38 52.0397) (width 0.6) (layer "B.Cu") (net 1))
 (segment (start 119.38 52.0397) (end 114.5606 47.2203) (width 0.6) (layer "B.Cu") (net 1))
 (segment (start 114.3 45.72) (end 114.3 47.2203) (width 0.6) (layer "B.Cu") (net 1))
 (segment (start 114.5606 47.2203) (end 114.3 47.2203) (width 0.6) (layer "B.Cu") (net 1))
 (segment (start 127.9663 90.9316) (end 136.0947 99.06) (width 0.6) (layer "B.Cu") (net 7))
 (segment (start 127.9663 69.5463) (end 127.9663 90.9316) (width 0.6) (layer "B.Cu") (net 7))
 (segment (start 121.285 62.865) (end 127.9663 69.5463) (width 0.6) (layer "B.Cu") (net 7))
 (segment (start 137.795 99.06) (end 136.0947 99.06) (width 0.6) (layer "B.Cu") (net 7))
 (segment (start 121.285 66.8053) (end 118.2367 69.8536) (width 0.6) (layer "B.Cu") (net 6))
 (segment (start 118.2367 69.8536) (end 118.2367 77.9783) (width 0.6) (layer "B.Cu") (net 6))
 (segment (start 121.285 65.405) (end 121.285 66.8053) (width 0.6) (layer "B.Cu") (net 6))
 (segment (start 118.2367 77.9783) (end 113.03 83.185) (width 0.6) (layer "B.Cu") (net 6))
 (segment (start 121.285 69.85) (end 123.9543 72.5193) (width 0.6) (layer "B.Cu") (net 9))
 (segment (start 123.9543 91.9996) (end 128.4747 96.52) (width 0.6) (layer "B.Cu") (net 9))
 (segment (start 130.175 96.52) (end 128.4747 96.52) (width 0.6) (layer "B.Cu") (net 9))
 (segment (start 123.9543 72.5193) (end 123.9543 91.9996) (width 0.6) (layer "B.Cu") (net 9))
 (segment (start 121.285 73.7903) (end 119.8847 75.1906) (width 0.6) (layer "B.Cu") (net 8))
 (segment (start 121.285 72.39) (end 121.285 73.7903) (width 0.6) (layer "B.Cu") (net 8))
 (segment (start 119.8847 78.8703) (end 113.03 85.725) (width 0.6) (layer "B.Cu") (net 8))
 (segment (start 119.8847 75.1906) (end 119.8847 78.8703) (width 0.6) (layer "B.Cu") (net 8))
 (segment (start 130.175 99.06) (end 128.4747 99.06) (width 0.6) (layer "F.Cu") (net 11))
 (segment (start 128.4747 87.9668) (end 128.4747 99.06) (width 0.6) (layer "F.Cu") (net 11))
 (segment (start 121.285 76.835) (end 125.7422 81.2922) (width 0.6) (layer "F.Cu") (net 11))
 (segment (start 125.7422 85.2343) (end 128.4747 87.9668) (width 0.6) (layer "F.Cu") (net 11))
 (segment (start 125.7422 81.2922) (end 125.7422 85.2343) (width 0.6) (layer "F.Cu") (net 11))
 (segment (start 121.285 79.375) (end 121.285 80.7753) (width 0.6) (layer "B.Cu") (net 10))
 (segment (start 113.03 88.265) (end 114.3303 88.265) (width 0.6) (layer "B.Cu") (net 10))
 (segment (start 114.3303 87.73) (end 114.3303 88.265) (width 0.6) (layer "B.Cu") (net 10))
 (segment (start 121.285 80.7753) (end 114.3303 87.73) (width 0.6) (layer "B.Cu") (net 10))
 (segment (start 125.8436 98.9689) (end 128.4747 101.6) (width 0.6) (layer "F.Cu") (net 21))
 (segment (start 130.175 101.6) (end 128.4747 101.6) (width 0.6) (layer "F.Cu") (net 21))
 (segment (start 125.8436 88.3786) (end 125.8436 98.9689) (width 0.6) (layer "F.Cu") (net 21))
 (segment (start 121.285 83.82) (end 125.8436 88.3786) (width 0.6) (layer "F.Cu") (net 21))
 (segment (start 121.285 86.36) (end 119.8847 86.36) (width 0.6) (layer "B.Cu") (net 20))
 (segment (start 115.4397 90.805) (end 113.03 90.805) (width 0.6) (layer "B.Cu") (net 20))
 (segment (start 119.8847 86.36) (end 115.4397 90.805) (width 0.6) (layer "B.Cu") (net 20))
 (segment (start 128.4747 97.9947) (end 128.4747 104.14) (width 0.6) (layer "B.Cu") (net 13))
 (segment (start 121.285 90.805) (end 128.4747 97.9947) (width 0.6) (layer "B.Cu") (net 13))
 (segment (start 130.175 104.14) (end 128.4747 104.14) (width 0.6) (layer "B.Cu") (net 13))
 (segment (start 121.285 93.345) (end 113.03 93.345) (width 0.6) (layer "B.Cu") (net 12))
 (segment (start 125.8436 102.3486) (end 125.8436 104.0489) (width 0.6) (layer "B.Cu") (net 15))
 (segment (start 121.285 97.79) (end 125.8436 102.3486) (width 0.6) (layer "B.Cu") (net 15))
 (segment (start 125.8436 104.0489) (end 128.4747 106.68) (width 0.6) (layer "B.Cu") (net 15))
 (segment (start 130.175 106.68) (end 128.4747 106.68) (width 0.6) (layer "B.Cu") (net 15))
 (segment (start 118.7753 100.33) (end 114.3303 95.885) (width 0.6) (layer "B.Cu") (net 14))
 (segment (start 121.285 100.33) (end 118.7753 100.33) (width 0.6) (layer "B.Cu") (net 14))
 (segment (start 113.03 95.885) (end 114.3303 95.885) (width 0.6) (layer "B.Cu") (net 14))
 (segment (start 121.285 104.775) (end 124.0297 104.775) (width 0.6) (layer "F.Cu") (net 17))
 (segment (start 124.0297 104.775) (end 128.4747 109.22) (width 0.6) (layer "F.Cu") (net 17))
 (segment (start 130.175 109.22) (end 128.4747 109.22) (width 0.6) (layer "F.Cu") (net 17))
 (segment (start 121.285 107.315) (end 113.03 99.06) (width 0.6) (layer "B.Cu") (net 16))
 (segment (start 113.03 99.06) (end 113.03 98.425) (width 0.6) (layer "B.Cu") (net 16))
 (segment (start 121.285 111.76) (end 130.175 111.76) (width 0.6) (layer "B.Cu") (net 19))
 (segment (start 121.285 114.3) (end 113.03 106.045) (width 0.6) (layer "B.Cu") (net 18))
 (segment (start 113.03 106.045) (end 113.03 100.965) (width 0.6) (layer "B.Cu") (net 18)))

